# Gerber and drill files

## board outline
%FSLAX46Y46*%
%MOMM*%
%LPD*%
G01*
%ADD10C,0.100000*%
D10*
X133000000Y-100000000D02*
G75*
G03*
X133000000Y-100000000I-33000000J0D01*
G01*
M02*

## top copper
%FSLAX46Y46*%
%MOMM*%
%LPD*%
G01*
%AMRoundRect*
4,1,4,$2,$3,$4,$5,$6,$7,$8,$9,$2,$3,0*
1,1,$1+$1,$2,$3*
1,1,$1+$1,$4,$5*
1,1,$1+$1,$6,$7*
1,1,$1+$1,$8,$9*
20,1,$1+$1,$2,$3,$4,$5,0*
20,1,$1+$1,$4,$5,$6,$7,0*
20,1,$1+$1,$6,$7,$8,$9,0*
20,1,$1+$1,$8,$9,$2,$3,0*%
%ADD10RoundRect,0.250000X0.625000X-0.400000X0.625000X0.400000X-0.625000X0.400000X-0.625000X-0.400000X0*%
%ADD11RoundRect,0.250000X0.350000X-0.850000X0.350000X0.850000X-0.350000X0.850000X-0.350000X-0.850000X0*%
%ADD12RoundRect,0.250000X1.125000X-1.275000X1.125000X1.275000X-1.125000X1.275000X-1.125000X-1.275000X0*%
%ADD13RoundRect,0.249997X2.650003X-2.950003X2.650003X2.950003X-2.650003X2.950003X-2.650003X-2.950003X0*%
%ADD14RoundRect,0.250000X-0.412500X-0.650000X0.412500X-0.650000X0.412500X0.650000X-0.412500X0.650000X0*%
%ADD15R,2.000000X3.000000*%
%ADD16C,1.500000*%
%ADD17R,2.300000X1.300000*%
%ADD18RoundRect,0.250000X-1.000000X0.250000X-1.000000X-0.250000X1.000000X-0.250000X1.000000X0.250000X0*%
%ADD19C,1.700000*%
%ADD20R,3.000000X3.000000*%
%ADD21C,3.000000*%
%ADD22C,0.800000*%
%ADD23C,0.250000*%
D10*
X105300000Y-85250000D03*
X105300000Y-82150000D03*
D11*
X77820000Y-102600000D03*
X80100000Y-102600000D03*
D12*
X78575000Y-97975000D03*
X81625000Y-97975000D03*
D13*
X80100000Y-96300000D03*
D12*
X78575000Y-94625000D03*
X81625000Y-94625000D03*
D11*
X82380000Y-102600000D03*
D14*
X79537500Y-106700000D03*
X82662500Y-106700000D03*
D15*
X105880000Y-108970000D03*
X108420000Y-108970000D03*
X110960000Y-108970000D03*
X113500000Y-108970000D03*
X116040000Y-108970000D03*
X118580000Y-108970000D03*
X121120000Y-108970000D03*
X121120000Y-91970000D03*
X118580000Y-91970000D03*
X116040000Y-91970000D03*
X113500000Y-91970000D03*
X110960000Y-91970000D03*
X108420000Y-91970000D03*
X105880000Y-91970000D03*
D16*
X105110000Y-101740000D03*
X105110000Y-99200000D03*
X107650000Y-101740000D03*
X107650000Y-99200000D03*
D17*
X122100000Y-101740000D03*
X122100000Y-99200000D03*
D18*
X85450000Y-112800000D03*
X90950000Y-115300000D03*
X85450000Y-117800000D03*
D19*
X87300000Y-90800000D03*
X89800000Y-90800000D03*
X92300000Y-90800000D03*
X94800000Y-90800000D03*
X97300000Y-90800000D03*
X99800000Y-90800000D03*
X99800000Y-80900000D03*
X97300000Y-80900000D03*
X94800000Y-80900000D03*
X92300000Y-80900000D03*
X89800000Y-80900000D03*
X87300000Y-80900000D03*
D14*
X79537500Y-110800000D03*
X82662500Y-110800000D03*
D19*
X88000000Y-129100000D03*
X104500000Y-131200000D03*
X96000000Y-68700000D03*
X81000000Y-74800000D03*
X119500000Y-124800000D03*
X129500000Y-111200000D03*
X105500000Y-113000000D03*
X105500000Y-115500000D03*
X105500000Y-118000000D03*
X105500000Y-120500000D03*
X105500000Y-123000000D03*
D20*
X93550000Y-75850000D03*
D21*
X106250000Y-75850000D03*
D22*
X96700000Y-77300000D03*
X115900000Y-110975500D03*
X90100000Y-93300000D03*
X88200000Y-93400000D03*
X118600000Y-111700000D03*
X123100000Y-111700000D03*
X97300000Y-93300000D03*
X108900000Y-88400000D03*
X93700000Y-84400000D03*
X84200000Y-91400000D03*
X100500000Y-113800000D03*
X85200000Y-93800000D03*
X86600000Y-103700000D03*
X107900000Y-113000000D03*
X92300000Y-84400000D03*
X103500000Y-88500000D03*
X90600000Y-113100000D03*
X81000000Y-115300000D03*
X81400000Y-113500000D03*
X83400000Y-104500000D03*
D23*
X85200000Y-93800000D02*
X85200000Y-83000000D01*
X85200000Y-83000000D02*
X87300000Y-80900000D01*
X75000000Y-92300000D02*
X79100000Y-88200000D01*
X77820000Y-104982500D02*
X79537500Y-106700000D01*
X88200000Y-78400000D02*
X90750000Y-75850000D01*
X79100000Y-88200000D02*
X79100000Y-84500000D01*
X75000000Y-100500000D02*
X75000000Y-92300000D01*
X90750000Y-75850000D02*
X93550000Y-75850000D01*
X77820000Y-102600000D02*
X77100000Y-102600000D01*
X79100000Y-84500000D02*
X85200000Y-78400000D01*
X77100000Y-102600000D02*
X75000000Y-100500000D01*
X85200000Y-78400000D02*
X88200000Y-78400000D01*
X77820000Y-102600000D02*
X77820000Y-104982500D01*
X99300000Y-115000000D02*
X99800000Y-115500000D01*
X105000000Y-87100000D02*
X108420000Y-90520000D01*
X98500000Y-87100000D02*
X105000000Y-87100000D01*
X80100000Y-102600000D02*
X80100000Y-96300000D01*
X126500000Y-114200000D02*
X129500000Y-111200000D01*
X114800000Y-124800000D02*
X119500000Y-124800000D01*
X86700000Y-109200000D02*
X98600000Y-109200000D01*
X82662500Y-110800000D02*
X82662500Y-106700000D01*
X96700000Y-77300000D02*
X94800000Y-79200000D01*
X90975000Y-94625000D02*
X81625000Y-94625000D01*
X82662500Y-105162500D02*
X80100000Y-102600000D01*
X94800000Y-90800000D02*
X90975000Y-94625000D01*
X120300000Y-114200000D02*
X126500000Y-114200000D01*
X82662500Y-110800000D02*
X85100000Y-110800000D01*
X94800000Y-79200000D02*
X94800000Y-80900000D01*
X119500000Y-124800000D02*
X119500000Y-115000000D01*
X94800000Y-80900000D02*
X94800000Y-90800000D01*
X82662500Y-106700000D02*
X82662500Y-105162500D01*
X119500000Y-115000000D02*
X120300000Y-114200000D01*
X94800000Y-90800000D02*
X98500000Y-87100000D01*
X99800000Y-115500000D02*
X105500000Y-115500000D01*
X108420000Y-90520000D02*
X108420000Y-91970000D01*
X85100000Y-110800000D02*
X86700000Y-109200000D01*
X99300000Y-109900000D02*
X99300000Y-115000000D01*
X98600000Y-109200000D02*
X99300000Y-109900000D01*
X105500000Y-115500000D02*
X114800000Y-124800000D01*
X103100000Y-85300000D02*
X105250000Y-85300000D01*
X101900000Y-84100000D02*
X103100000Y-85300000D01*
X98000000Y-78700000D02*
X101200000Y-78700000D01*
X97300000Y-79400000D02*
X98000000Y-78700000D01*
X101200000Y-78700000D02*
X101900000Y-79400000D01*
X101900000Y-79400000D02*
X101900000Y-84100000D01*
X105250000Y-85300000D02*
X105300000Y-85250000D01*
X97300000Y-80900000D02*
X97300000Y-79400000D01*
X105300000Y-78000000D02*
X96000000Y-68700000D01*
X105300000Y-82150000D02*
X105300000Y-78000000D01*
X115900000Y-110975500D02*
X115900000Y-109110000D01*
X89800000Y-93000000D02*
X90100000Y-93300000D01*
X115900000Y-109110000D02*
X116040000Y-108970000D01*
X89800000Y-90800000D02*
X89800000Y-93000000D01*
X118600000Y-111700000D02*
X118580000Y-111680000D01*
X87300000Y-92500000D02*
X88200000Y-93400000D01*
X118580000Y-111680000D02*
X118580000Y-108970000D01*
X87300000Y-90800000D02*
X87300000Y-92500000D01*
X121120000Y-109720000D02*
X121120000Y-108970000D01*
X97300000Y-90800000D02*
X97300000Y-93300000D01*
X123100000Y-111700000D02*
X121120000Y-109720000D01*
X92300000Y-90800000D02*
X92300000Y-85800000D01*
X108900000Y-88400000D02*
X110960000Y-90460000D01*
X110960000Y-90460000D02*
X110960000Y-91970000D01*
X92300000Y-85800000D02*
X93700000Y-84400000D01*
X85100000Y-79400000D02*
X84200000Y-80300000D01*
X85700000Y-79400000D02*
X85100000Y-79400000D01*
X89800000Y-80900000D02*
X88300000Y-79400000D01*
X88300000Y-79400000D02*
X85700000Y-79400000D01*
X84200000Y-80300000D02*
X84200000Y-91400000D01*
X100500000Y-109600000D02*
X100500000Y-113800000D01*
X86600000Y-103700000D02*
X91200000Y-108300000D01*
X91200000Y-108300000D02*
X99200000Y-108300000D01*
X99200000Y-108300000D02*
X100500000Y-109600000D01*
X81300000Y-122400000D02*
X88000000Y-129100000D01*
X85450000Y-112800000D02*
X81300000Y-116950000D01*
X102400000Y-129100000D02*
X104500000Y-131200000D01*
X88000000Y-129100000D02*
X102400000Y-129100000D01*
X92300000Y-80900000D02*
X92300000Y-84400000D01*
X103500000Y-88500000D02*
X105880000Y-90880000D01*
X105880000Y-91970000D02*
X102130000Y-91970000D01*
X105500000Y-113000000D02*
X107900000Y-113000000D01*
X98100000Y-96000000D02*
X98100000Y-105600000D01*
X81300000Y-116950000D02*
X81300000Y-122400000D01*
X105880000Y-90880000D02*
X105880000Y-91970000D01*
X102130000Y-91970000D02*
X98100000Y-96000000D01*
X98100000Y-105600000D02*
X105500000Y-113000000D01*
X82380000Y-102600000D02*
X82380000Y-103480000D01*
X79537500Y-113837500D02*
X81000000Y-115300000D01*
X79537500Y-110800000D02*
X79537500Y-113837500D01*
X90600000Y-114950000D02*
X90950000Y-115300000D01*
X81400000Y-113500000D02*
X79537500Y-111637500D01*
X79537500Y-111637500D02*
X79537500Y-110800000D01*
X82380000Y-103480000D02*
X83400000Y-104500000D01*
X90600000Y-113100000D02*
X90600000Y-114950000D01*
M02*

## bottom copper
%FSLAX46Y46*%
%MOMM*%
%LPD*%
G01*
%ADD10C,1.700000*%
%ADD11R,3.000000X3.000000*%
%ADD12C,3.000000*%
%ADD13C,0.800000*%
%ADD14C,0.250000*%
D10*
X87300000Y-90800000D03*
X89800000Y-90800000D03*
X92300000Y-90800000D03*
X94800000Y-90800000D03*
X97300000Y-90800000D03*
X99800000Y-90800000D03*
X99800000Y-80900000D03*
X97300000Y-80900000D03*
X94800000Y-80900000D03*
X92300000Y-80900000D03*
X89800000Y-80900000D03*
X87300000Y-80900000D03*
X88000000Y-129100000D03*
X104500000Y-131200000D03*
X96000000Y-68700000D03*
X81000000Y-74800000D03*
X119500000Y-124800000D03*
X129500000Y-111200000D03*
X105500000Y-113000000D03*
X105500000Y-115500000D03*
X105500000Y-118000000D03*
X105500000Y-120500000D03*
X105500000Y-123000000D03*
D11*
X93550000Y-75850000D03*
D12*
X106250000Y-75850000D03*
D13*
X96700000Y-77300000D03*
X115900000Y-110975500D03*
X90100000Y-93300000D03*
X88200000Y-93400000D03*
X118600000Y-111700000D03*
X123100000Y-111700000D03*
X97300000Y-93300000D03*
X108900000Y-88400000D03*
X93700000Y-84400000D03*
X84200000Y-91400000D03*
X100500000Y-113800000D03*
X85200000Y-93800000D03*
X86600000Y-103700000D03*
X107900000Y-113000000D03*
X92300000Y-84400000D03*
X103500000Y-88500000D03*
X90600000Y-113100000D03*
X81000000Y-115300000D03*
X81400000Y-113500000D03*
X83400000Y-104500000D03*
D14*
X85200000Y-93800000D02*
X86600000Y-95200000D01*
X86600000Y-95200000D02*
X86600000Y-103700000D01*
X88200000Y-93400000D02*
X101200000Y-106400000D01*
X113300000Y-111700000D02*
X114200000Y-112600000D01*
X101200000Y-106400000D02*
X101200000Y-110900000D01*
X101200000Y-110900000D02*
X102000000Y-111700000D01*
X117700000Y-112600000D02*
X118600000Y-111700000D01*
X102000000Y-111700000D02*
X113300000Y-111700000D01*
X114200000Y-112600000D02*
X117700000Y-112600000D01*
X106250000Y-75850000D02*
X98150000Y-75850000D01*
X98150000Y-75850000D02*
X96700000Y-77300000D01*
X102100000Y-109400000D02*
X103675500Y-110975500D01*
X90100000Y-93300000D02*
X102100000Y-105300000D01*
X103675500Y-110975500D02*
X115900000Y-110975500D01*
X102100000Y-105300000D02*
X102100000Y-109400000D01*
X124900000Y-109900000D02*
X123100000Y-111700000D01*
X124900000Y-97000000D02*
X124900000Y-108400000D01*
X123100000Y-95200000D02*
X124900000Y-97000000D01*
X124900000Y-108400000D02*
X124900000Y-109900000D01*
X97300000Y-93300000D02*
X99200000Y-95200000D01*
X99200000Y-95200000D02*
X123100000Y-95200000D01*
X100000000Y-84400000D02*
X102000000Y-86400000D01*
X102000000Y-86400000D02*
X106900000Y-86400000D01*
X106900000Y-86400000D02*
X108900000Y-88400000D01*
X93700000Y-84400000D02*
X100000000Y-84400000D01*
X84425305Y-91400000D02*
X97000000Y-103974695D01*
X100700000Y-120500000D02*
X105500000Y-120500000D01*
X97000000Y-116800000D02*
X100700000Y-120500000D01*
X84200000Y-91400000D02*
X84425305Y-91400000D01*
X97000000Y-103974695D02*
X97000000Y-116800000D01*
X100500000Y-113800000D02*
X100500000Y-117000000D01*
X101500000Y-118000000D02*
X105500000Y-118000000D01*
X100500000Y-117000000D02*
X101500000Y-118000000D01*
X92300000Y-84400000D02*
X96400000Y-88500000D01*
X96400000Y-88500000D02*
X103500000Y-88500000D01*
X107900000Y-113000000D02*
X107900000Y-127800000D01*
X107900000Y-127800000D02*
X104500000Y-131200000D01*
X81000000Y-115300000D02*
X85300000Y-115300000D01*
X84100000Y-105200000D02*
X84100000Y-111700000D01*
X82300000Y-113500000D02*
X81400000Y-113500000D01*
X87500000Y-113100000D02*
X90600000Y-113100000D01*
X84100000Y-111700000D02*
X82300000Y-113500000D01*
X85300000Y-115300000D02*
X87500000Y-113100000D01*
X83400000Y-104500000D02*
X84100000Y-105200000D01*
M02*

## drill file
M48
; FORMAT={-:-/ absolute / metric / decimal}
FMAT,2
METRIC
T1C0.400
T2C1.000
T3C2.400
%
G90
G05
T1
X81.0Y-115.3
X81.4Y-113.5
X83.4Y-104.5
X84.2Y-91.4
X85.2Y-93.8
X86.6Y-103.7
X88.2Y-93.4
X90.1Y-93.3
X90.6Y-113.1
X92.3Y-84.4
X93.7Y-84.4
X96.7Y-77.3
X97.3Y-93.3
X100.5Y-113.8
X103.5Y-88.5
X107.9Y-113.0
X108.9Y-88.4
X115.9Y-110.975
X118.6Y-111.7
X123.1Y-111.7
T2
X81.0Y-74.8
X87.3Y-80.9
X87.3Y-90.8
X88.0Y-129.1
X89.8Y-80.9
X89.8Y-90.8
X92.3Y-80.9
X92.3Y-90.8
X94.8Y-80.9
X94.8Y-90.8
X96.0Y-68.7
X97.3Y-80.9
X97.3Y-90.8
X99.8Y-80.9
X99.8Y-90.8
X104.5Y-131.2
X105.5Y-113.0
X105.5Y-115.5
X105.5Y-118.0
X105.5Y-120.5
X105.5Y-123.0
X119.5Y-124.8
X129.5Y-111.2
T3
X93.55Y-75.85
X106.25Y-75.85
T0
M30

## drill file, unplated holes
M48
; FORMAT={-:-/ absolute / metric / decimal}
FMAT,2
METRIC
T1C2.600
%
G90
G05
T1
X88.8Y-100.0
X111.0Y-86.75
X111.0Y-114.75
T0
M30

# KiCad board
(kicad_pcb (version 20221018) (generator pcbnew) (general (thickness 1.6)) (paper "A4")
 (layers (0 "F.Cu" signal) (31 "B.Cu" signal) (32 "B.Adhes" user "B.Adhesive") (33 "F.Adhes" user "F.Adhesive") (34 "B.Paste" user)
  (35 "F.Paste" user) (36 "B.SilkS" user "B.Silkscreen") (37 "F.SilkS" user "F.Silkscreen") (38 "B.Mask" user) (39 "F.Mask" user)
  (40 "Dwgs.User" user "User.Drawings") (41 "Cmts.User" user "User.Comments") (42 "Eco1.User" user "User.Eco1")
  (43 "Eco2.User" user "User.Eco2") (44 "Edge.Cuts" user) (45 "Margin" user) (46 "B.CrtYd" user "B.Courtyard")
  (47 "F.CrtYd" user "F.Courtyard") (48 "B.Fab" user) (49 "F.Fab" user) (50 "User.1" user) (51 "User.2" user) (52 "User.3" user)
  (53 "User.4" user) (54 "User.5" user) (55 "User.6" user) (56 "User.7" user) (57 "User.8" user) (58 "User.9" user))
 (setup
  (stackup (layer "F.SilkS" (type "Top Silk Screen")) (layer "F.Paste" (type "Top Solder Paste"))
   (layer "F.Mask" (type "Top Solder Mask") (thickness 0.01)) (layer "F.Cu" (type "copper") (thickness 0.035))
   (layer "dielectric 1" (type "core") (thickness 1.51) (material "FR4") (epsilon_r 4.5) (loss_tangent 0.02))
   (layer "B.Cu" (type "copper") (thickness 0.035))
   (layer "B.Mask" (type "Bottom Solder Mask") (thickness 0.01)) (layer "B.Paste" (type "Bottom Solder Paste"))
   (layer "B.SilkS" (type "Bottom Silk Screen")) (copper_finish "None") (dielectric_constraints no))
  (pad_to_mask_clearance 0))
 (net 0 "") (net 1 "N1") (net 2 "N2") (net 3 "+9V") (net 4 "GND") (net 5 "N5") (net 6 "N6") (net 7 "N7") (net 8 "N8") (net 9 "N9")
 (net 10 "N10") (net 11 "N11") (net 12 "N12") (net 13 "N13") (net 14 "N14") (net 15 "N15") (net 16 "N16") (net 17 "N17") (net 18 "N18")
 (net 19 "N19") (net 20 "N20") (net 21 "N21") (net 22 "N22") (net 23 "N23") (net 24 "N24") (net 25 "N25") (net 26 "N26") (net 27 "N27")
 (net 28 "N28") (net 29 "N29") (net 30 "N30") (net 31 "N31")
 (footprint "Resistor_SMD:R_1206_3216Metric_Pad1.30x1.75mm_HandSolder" (layer "F.Cu") (at 105.3 83.7 90)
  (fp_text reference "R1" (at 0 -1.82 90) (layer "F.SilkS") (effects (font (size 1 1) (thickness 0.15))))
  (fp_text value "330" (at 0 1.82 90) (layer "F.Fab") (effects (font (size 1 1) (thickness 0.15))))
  (pad "1" smd roundrect (at -1.55 0 90) (size 1.3 1.75) (layers "F.Cu" "F.Paste" "F.Mask") (roundrect_rratio 0.1923076923) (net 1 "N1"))
  (pad "2" smd roundrect (at 1.55 0 90) (size 1.3 1.75) (layers "F.Cu" "F.Paste" "F.Mask") (roundrect_rratio 0.1923076923) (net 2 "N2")))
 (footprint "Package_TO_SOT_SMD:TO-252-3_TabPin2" (layer "F.Cu") (at 80.1 97.56 90)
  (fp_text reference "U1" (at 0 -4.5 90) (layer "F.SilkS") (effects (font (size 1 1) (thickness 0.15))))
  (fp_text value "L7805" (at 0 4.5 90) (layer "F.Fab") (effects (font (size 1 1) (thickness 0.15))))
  (pad "1" smd roundrect (at -5.04 -2.28 90) (size 2.2 1.2) (layers "F.Cu" "F.Paste" "F.Mask") (roundrect_rratio 0.2083333333) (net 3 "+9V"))
  (pad "2" smd roundrect (at -5.04 0 90) (size 2.2 1.2) (layers "F.Cu" "F.Paste" "F.Mask") (roundrect_rratio 0.2083333333) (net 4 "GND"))
  (pad "2" smd roundrect (at -0.415 -1.525 90) (size 3.05 2.75) (layers "F.Cu" "F.Paste") (roundrect_rratio 0.09090909091) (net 4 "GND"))
  (pad "2" smd roundrect (at -0.415 1.525 90) (size 3.05 2.75) (layers "F.Cu" "F.Paste") (roundrect_rratio 0.09090909091) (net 4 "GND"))
  (pad "2" smd roundrect (at 1.26 0 90) (size 6.4 5.8) (layers "F.Cu" "F.Mask") (roundrect_rratio 0.04310293103) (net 4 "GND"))
  (pad "2" smd roundrect (at 2.935 -1.525 90) (size 3.05 2.75) (layers "F.Cu" "F.Paste") (roundrect_rratio 0.09090909091) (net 4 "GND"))
  (pad "2" smd roundrect (at 2.935 1.525 90) (size 3.05 2.75) (layers "F.Cu" "F.Paste") (roundrect_rratio 0.09090909091) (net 4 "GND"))
  (pad "3" smd roundrect (at -5.04 2.28 90) (size 2.2 1.2) (layers "F.Cu" "F.Paste" "F.Mask") (roundrect_rratio 0.2083333333) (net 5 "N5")))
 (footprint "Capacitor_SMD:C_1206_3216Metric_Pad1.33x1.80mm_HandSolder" (layer "F.Cu") (at 81.1 106.7)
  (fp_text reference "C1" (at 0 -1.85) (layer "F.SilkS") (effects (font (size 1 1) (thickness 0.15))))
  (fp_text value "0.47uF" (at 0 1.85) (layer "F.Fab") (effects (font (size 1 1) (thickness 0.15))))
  (pad "1" smd roundrect (at -1.5625 0) (size 1.325 1.8) (layers "F.Cu" "F.Paste" "F.Mask") (roundrect_rratio 0.1886792453) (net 3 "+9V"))
  (pad "2" smd roundrect (at 1.5625 0) (size 1.325 1.8) (layers "F.Cu" "F.Paste" "F.Mask") (roundrect_rratio 0.1886792453) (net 4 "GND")))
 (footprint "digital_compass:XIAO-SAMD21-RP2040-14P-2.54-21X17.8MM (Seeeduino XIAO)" (layer "F.Cu") (at 113.5 100.47 90)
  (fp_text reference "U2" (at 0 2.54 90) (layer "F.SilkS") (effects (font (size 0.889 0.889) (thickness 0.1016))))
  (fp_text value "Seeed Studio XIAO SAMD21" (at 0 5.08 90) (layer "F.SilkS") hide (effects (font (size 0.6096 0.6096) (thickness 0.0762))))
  (pad "1" smd rect (at -8.5 -7.62 90) (size 3 2) (layers "F.Cu" "F.Paste" "F.Mask") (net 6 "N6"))
  (pad "2" smd rect (at -8.5 -5.08 90) (size 3 2) (layers "F.Cu" "F.Paste" "F.Mask") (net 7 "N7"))
  (pad "3" smd rect (at -8.5 -2.54 90) (size 3 2) (layers "F.Cu" "F.Paste" "F.Mask") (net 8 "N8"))
  (pad "4" smd rect (at -8.5 0 90) (size 3 2) (layers "F.Cu" "F.Paste" "F.Mask") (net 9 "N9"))
  (pad "5" smd rect (at -8.5 2.54 90) (size 3 2) (layers "F.Cu" "F.Paste" "F.Mask") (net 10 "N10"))
  (pad "6" smd rect (at -8.5 5.08 270) (size 3 2) (layers "F.Cu" "F.Paste" "F.Mask") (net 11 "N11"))
  (pad "7" smd rect (at -8.5 7.62 90) (size 3 2) (layers "F.Cu" "F.Paste" "F.Mask") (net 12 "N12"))
  (pad "8" smd rect (at 8.5 7.62 90) (size 3 2) (layers "F.Cu" "F.Paste" "F.Mask") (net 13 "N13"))
  (pad "9" smd rect (at 8.5 5.08 90) (size 3 2) (layers "F.Cu" "F.Paste" "F.Mask") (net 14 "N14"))
  (pad "10" smd rect (at 8.5 2.54 90) (size 3 2) (layers "F.Cu" "F.Paste" "F.Mask") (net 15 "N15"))
  (pad "11" smd rect (at 8.5 0 90) (size 3 2) (layers "F.Cu" "F.Paste" "F.Mask") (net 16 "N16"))
  (pad "12" smd rect (at 8.5 -2.54 90) (size 3 2) (layers "F.Cu" "F.Paste" "F.Mask") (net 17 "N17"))
  (pad "13" smd rect (at 8.5 -5.08 90) (size 3 2) (layers "F.Cu" "F.Paste" "F.Mask") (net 4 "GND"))
  (pad "14" smd rect (at 8.5 -7.62 90) (size 3 2) (layers "F.Cu" "F.Paste" "F.Mask") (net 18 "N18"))
  (pad "15" smd circle (at -1.27 -8.39 180) (size 1.5 1.5) (layers "F.Cu" "F.Paste" "F.Mask") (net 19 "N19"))
  (pad "16" smd circle (at 1.27 -8.39 180) (size 1.5 1.5) (layers "F.Cu" "F.Paste" "F.Mask") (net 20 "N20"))
  (pad "17" smd circle (at -1.27 -5.85 180) (size 1.5 1.5) (layers "F.Cu" "F.Paste" "F.Mask") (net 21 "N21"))
  (pad "18" smd circle (at 1.27 -5.85 180) (size 1.5 1.5) (layers "F.Cu" "F.Paste" "F.Mask") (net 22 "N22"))
  (pad "19" smd rect (at -1.27 8.6 180) (size 2.3 1.3) (layers "F.Cu" "F.Paste" "F.Mask") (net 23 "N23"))
  (pad "20" smd rect (at 1.27 8.6 180) (size 2.3 1.3) (layers "F.Cu" "F.Paste" "F.Mask") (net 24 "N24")))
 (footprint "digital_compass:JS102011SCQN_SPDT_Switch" (layer "F.Cu") (at 88.2 115.3 -90)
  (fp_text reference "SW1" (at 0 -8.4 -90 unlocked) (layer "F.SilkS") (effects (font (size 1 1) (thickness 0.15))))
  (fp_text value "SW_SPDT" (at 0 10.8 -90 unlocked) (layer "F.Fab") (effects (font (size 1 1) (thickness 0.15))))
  (pad "1" smd roundrect (at -2.5 2.75 270) (size 1 2.5) (layers "F.Cu" "F.Paste" "F.Mask") (roundrect_rratio 0.25) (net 18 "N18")
   (thermal_bridge_angle 45))
  (pad "2" smd roundrect (at 0 -2.75 270) (size 1 2.5) (layers "F.Cu" "F.Paste" "F.Mask") (roundrect_rratio 0.25) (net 5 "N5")
   (thermal_bridge_angle 45))
  (pad "3" smd roundrect (at 2.5 2.75 270) (size 1 2.5) (layers "F.Cu" "F.Paste" "F.Mask") (roundrect_rratio 0.25) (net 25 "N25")
   (thermal_bridge_angle 45)))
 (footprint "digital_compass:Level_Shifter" (layer "F.Cu") (at 93.55 85.85)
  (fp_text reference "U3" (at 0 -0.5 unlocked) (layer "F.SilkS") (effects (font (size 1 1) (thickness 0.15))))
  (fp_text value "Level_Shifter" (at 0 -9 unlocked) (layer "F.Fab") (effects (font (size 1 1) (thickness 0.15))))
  (pad "1" thru_hole circle (at -6.25 4.95) (size 1.7 1.7) (drill 1) (layers "*.Cu" "*.Mask") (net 11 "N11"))
  (pad "2" thru_hole circle (at -3.75 4.95) (size 1.7 1.7) (drill 1) (layers "*.Cu" "*.Mask") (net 10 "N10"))
  (pad "3" thru_hole circle (at -1.25 4.95) (size 1.7 1.7) (drill 1) (layers "*.Cu" "*.Mask") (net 17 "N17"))
  (pad "4" thru_hole circle (at 1.25 4.95) (size 1.7 1.7) (drill 1) (layers "*.Cu" "*.Mask") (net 4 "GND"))
  (pad "5" thru_hole circle (at 3.75 4.95) (size 1.7 1.7) (drill 1) (layers "*.Cu" "*.Mask") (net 12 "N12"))
  (pad "6" thru_hole circle (at 6.25 4.95) (size 1.7 1.7) (drill 1) (layers "*.Cu" "*.Mask") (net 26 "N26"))
  (pad "7" thru_hole circle (at 6.25 -4.95) (size 1.7 1.7) (drill 1) (layers "*.Cu" "*.Mask") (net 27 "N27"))
  (pad "8" thru_hole circle (at 3.75 -4.95) (size 1.7 1.7) (drill 1) (layers "*.Cu" "*.Mask") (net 1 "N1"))
  (pad "9" thru_hole circle (at 1.25 -4.95) (size 1.7 1.7) (drill 1) (layers "*.Cu" "*.Mask") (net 4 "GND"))
  (pad "10" thru_hole circle (at -1.25 -4.95) (size 1.7 1.7) (drill 1) (layers "*.Cu" "*.Mask") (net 18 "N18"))
  (pad "11" thru_hole circle (at -3.75 -4.95) (size 1.7 1.7) (drill 1) (layers "*.Cu" "*.Mask") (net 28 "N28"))
  (pad "12" thru_hole circle (at -6.25 -4.95) (size 1.7 1.7) (drill 1) (layers "*.Cu" "*.Mask") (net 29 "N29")))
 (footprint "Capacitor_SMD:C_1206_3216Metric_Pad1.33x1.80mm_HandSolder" (layer "F.Cu") (at 81.1 110.8)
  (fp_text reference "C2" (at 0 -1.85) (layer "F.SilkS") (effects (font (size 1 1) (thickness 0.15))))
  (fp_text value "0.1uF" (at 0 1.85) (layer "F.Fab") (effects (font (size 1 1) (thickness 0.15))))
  (pad "1" smd roundrect (at -1.5625 0) (size 1.325 1.8) (layers "F.Cu" "F.Paste" "F.Mask") (roundrect_rratio 0.1886792453) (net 5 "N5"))
  (pad "2" smd roundrect (at 1.5625 0) (size 1.325 1.8) (layers "F.Cu" "F.Paste" "F.Mask") (roundrect_rratio 0.1886792453) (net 4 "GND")))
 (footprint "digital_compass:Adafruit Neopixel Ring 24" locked (layer "F.Cu") (at 100 100)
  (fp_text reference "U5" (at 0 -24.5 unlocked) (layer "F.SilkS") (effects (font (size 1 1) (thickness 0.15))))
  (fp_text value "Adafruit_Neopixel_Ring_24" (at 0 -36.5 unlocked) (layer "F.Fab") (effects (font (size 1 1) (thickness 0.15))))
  (pad "1" thru_hole circle locked (at -12 29.1) (size 1.7 1.7) (drill 1) (layers "*.Cu" "*.Mask") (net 18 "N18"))
  (pad "2" thru_hole circle locked (at 4.5 31.2) (size 1.7 1.7) (drill 1) (layers "*.Cu" "*.Mask") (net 18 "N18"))
  (pad "3" thru_hole circle locked (at -4 -31.3) (size 1.7 1.7) (drill 1) (layers "*.Cu" "*.Mask") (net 2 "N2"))
  (pad "4" thru_hole circle locked (at -19 -25.2) (size 1.7 1.7) (drill 1) (layers "*.Cu" "*.Mask") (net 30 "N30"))
  (pad "5" thru_hole circle locked (at 19.5 24.8) (size 1.7 1.7) (drill 1) (layers "*.Cu" "*.Mask") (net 4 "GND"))
  (pad "6" thru_hole circle locked (at 29.5 11.2) (size 1.7 1.7) (drill 1) (layers "*.Cu" "*.Mask") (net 4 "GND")))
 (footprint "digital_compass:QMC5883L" (layer "F.Cu") (at 100 118)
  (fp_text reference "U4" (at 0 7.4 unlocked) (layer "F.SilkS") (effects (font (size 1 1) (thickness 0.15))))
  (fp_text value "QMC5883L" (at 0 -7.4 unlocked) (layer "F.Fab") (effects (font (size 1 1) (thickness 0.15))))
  (pad "1" thru_hole circle (at 5.5 -5) (size 1.7 1.7) (drill 1) (layers "*.Cu" "*.Mask") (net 18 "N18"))
  (pad "2" thru_hole circle (at 5.5 -2.5) (size 1.7 1.7) (drill 1) (layers "*.Cu" "*.Mask") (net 4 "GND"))
  (pad "3" thru_hole circle (at 5.5 0) (size 1.7 1.7) (drill 1) (layers "*.Cu" "*.Mask") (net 29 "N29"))
  (pad "4" thru_hole circle (at 5.5 2.5) (size 1.7 1.7) (drill 1) (layers "*.Cu" "*.Mask") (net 28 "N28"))
  (pad "5" thru_hole circle (at 5.5 5) (size 1.7 1.7) (drill 1) (layers "*.Cu" "*.Mask") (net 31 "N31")))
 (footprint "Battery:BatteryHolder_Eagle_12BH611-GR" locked (layer "B.Cu") (at 93.55 75.85 90)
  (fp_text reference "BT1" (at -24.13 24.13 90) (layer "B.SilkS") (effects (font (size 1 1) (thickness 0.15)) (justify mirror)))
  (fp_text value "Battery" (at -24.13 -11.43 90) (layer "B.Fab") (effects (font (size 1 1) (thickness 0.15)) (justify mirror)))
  (pad "" np_thru_hole circle locked (at -38.9 17.45 90) (size 2.6 2.6) (drill 2.6) (layers "*.Cu" "*.Mask"))
  (pad "" np_thru_hole circle locked (at -24.15 -4.75 90) (size 2.6 2.6) (drill 2.6) (layers "*.Cu" "*.Mask"))
  (pad "" np_thru_hole circle locked (at -10.9 17.45 90) (size 2.6 2.6) (drill 2.6) (layers "*.Cu" "*.Mask"))
  (pad "1" thru_hole rect locked (at 0 0 90) (size 3 3) (drill 2.4) (layers "*.Cu" "*.Mask") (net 3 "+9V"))
  (pad "2" thru_hole circle locked (at 0 12.7 90) (size 3 3) (drill 2.4) (layers "*.Cu" "*.Mask") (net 4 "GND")))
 (gr_circle (center 100 100) (end 133 100) (stroke (width 0.1) (type default)) (fill none) (layer "Edge.Cuts"))
 (segment (start 75 92.3) (end 79.1 88.2) (width 0.25) (layer "F.Cu") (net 3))
 (segment (start 77.82 104.9825) (end 79.5375 106.7) (width 0.25) (layer "F.Cu") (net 3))
 (segment (start 88.2 78.4) (end 90.75 75.85) (width 0.25) (layer "F.Cu") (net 3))
 (segment (start 79.1 88.2) (end 79.1 84.5) (width 0.25) (layer "F.Cu") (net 3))
 (segment (start 75 100.5) (end 75 92.3) (width 0.25) (layer "F.Cu") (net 3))
 (segment (start 90.75 75.85) (end 93.55 75.85) (width 0.25) (layer "F.Cu") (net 3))
 (segment (start 77.82 102.6) (end 77.1 102.6) (width 0.25) (layer "F.Cu") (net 3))
 (segment (start 79.1 84.5) (end 85.2 78.4) (width 0.25) (layer "F.Cu") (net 3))
 (segment (start 77.1 102.6) (end 75 100.5) (width 0.25) (layer "F.Cu") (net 3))
 (segment (start 85.2 78.4) (end 88.2 78.4) (width 0.25) (layer "F.Cu") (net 3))
 (segment (start 77.82 102.6) (end 77.82 104.9825) (width 0.25) (layer "F.Cu") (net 3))
 (segment (start 99.3 115) (end 99.8 115.5) (width 0.25) (layer "F.Cu") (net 4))
 (segment (start 105 87.1) (end 108.42 90.52) (width 0.25) (layer "F.Cu") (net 4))
 (segment (start 98.5 87.1) (end 105 87.1) (width 0.25) (layer "F.Cu") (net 4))
 (segment (start 80.1 102.6) (end 80.1 96.3) (width 0.25) (layer "F.Cu") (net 4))
 (segment (start 126.5 114.2) (end 129.5 111.2) (width 0.25) (layer "F.Cu") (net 4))
 (segment (start 114.8 124.8) (end 119.5 124.8) (width 0.25) (layer "F.Cu") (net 4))
 (segment (start 86.7 109.2) (end 98.6 109.2) (width 0.25) (layer "F.Cu") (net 4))
 (segment (start 82.6625 110.8) (end 82.6625 106.7) (width 0.25) (layer "F.Cu") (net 4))
 (segment (start 96.7 77.3) (end 94.8 79.2) (width 0.25) (layer "F.Cu") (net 4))
 (segment (start 90.975 94.625) (end 81.625 94.625) (width 0.25) (layer "F.Cu") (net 4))
 (segment (start 82.6625 105.1625) (end 80.1 102.6) (width 0.25) (layer "F.Cu") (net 4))
 (segment (start 94.8 90.8) (end 90.975 94.625) (width 0.25) (layer "F.Cu") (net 4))
 (segment (start 120.3 114.2) (end 126.5 114.2) (width 0.25) (layer "F.Cu") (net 4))
 (segment (start 82.6625 110.8) (end 85.1 110.8) (width 0.25) (layer "F.Cu") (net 4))
 (segment (start 94.8 79.2) (end 94.8 80.9) (width 0.25) (layer "F.Cu") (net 4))
 (segment (start 119.5 124.8) (end 119.5 115) (width 0.25) (layer "F.Cu") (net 4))
 (segment (start 94.8 80.9) (end 94.8 90.8) (width 0.25) (layer "F.Cu") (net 4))
 (segment (start 82.6625 106.7) (end 82.6625 105.1625) (width 0.25) (layer "F.Cu") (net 4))
 (segment (start 119.5 115) (end 120.3 114.2) (width 0.25) (layer "F.Cu") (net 4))
 (segment (start 94.8 90.8) (end 98.5 87.1) (width 0.25) (layer "F.Cu") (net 4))
 (segment (start 99.8 115.5) (end 105.5 115.5) (width 0.25) (layer "F.Cu") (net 4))
 (segment (start 108.42 90.52) (end 108.42 91.97) (width 0.25) (layer "F.Cu") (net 4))
 (segment (start 85.1 110.8) (end 86.7 109.2) (width 0.25) (layer "F.Cu") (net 4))
 (segment (start 99.3 109.9) (end 99.3 115) (width 0.25) (layer "F.Cu") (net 4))
 (segment (start 98.6 109.2) (end 99.3 109.9) (width 0.25) (layer "F.Cu") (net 4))
 (segment (start 105.5 115.5) (end 114.8 124.8) (width 0.25) (layer "F.Cu") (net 4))
 (via (at 96.7 77.3) (size 0.8) (drill 0.4) (layers "F.Cu" "B.Cu") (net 4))
 (segment (start 106.25 75.85) (end 98.15 75.85) (width 0.25) (layer "B.Cu") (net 4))
 (segment (start 98.15 75.85) (end 96.7 77.3) (width 0.25) (layer "B.Cu") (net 4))
 (segment (start 103.1 85.3) (end 105.25 85.3) (width 0.25) (layer "F.Cu") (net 1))
 (segment (start 101.9 84.1) (end 103.1 85.3) (width 0.25) (layer "F.Cu") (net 1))
 (segment (start 98 78.7) (end 101.2 78.7) (width 0.25) (layer "F.Cu") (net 1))
 (segment (start 97.3 79.4) (end 98 78.7) (width 0.25) (layer "F.Cu") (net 1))
 (segment (start 101.2 78.7) (end 101.9 79.4) (width 0.25) (layer "F.Cu") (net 1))
 (segment (start 101.9 79.4) (end 101.9 84.1) (width 0.25) (layer "F.Cu") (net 1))
 (segment (start 105.25 85.3) (end 105.3 85.25) (width 0.25) (layer "F.Cu") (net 1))
 (segment (start 97.3 80.9) (end 97.3 79.4) (width 0.25) (layer "F.Cu") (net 1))
 (segment (start 105.3 78) (end 96 68.7) (width 0.25) (layer "F.Cu") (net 2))
 (segment (start 105.3 82.15) (end 105.3 78) (width 0.25) (layer "F.Cu") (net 2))
 (segment (start 115.9 110.9755) (end 115.9 109.11) (width 0.25) (layer "F.Cu") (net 10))
 (segment (start 89.8 93) (end 90.1 93.3) (width 0.25) (layer "F.Cu") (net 10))
 (segment (start 115.9 109.11) (end 116.04 108.97) (width 0.25) (layer "F.Cu") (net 10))
 (segment (start 89.8 90.8) (end 89.8 93) (width 0.25) (layer "F.Cu") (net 10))
 (via (at 115.9 110.9755) (size 0.8) (drill 0.4) (layers "F.Cu" "B.Cu") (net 10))
 (via (at 90.1 93.3) (size 0.8) (drill 0.4) (layers "F.Cu" "B.Cu") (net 10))
 (segment (start 102.1 109.4) (end 103.6755 110.9755) (width 0.25) (layer "B.Cu") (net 10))
 (segment (start 90.1 93.3) (end 102.1 105.3) (width 0.25) (layer "B.Cu") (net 10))
 (segment (start 103.6755 110.9755) (end 115.9 110.9755) (width 0.25) (layer "B.Cu") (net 10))
 (segment (start 102.1 105.3) (end 102.1 109.4) (width 0.25) (layer "B.Cu") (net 10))
 (segment (start 118.6 111.7) (end 118.58 111.68) (width 0.25) (layer "F.Cu") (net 11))
 (segment (start 87.3 92.5) (end 88.2 93.4) (width 0.25) (layer "F.Cu") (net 11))
 (segment (start 118.58 111.68) (end 118.58 108.97) (width 0.25) (layer "F.Cu") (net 11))
 (segment (start 87.3 90.8) (end 87.3 92.5) (width 0.25) (layer "F.Cu") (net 11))
 (via (at 88.2 93.4) (size 0.8) (drill 0.4) (layers "F.Cu" "B.Cu") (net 11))
 (via (at 118.6 111.7) (size 0.8) (drill 0.4) (layers "F.Cu" "B.Cu") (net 11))
 (segment (start 117.7 112.6) (end 118.6 111.7) (width 0.25) (layer "B.Cu") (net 11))
 (segment (start 101.2 106.4) (end 101.2 110.9) (width 0.25) (layer "B.Cu") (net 11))
 (segment (start 114.2 112.6) (end 117.7 112.6) (width 0.25) (layer "B.Cu") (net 11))
 (segment (start 101.2 110.9) (end 102 111.7) (width 0.25) (layer "B.Cu") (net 11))
 (segment (start 113.3 111.7) (end 114.2 112.6) (width 0.25) (layer "B.Cu") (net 11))
 (segment (start 88.2 93.4) (end 101.2 106.4) (width 0.25) (layer "B.Cu") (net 11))
 (segment (start 102 111.7) (end 113.3 111.7) (width 0.25) (layer "B.Cu") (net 11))
 (segment (start 121.12 109.72) (end 121.12 108.97) (width 0.25) (layer "F.Cu") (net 12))
 (segment (start 97.3 90.8) (end 97.3 93.3) (width 0.25) (layer "F.Cu") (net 12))
 (segment (start 123.1 111.7) (end 121.12 109.72) (width 0.25) (layer "F.Cu") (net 12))
 (via (at 123.1 111.7) (size 0.8) (drill 0.4) (layers "F.Cu" "B.Cu") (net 12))
 (via (at 97.3 93.3) (size 0.8) (drill 0.4) (layers "F.Cu" "B.Cu") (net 12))
 (segment (start 124.9 109.9) (end 123.1 111.7) (width 0.25) (layer "B.Cu") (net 12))
 (segment (start 124.9 97) (end 124.9 108.4) (width 0.25) (layer "B.Cu") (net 12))
 (segment (start 123.1 95.2) (end 124.9 97) (width 0.25) (layer "B.Cu") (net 12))
 (segment (start 124.9 108.4) (end 124.9 109.9) (width 0.25) (layer "B.Cu") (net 12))
 (segment (start 97.3 93.3) (end 99.2 95.2) (width 0.25) (layer "B.Cu") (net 12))
 (segment (start 99.2 95.2) (end 123.1 95.2) (width 0.25) (layer "B.Cu") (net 12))
 (segment (start 92.3 90.8) (end 92.3 85.8) (width 0.25) (layer "F.Cu") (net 17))
 (segment (start 108.9 88.4) (end 110.96 90.46) (width 0.25) (layer "F.Cu") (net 17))
 (segment (start 110.96 90.46) (end 110.96 91.97) (width 0.25) (layer "F.Cu") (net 17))
 (segment (start 92.3 85.8) (end 93.7 84.4) (width 0.25) (layer "F.Cu") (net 17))
 (via (at 108.9 88.4) (size 0.8) (drill 0.4) (layers "F.Cu" "B.Cu") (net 17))
 (via (at 93.7 84.4) (size 0.8) (drill 0.4) (layers "F.Cu" "B.Cu") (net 17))
 (segment (start 100 84.4) (end 102 86.4) (width 0.25) (layer "B.Cu") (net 17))
 (segment (start 102 86.4) (end 106.9 86.4) (width 0.25) (layer "B.Cu") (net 17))
 (segment (start 106.9 86.4) (end 108.9 88.4) (width 0.25) (layer "B.Cu") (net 17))
 (segment (start 93.7 84.4) (end 100 84.4) (width 0.25) (layer "B.Cu") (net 17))
 (segment (start 85.1 79.4) (end 84.2 80.3) (width 0.25) (layer "F.Cu") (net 28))
 (segment (start 85.7 79.4) (end 85.1 79.4) (width 0.25) (layer "F.Cu") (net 28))
 (segment (start 89.8 80.9) (end 88.3 79.4) (width 0.25) (layer "F.Cu") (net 28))
 (segment (start 88.3 79.4) (end 85.7 79.4) (width 0.25) (layer "F.Cu") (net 28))
 (segment (start 84.2 80.3) (end 84.2 91.4) (width 0.25) (layer "F.Cu") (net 28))
 (via (at 84.2 91.4) (size 0.8) (drill 0.4) (layers "F.Cu" "B.Cu") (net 28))
 (segment (start 84.425305 91.4) (end 97 103.974695) (width 0.25) (layer "B.Cu") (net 28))
 (segment (start 100.7 120.5) (end 105.5 120.5) (width 0.25) (layer "B.Cu") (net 28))
 (segment (start 97 116.8) (end 100.7 120.5) (width 0.25) (layer "B.Cu") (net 28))
 (segment (start 84.2 91.4) (end 84.425305 91.4) (width 0.25) (layer "B.Cu") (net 28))
 (segment (start 97 103.974695) (end 97 116.8) (width 0.25) (layer "B.Cu") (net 28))
 (segment (start 100.5 109.6) (end 100.5 113.8) (width 0.25) (layer "F.Cu") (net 29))
 (segment (start 86.6 103.7) (end 91.2 108.3) (width 0.25) (layer "F.Cu") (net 29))
 (segment (start 91.2 108.3) (end 99.2 108.3) (width 0.25) (layer "F.Cu") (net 29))
 (segment (start 99.2 108.3) (end 100.5 109.6) (width 0.25) (layer "F.Cu") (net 29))
 (segment (start 85.2 93.8) (end 85.2 83) (width 0.25) (layer "F.Cu") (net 29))
 (segment (start 85.2 83) (end 87.3 80.9) (width 0.25) (layer "F.Cu") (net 29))
 (via (at 100.5 113.8) (size 0.8) (drill 0.4) (layers "F.Cu" "B.Cu") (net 29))
 (via (at 85.2 93.8) (size 0.8) (drill 0.4) (layers "F.Cu" "B.Cu") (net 29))
 (via (at 86.6 103.7) (size 0.8) (drill 0.4) (layers "F.Cu" "B.Cu") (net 29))
 (segment (start 85.2 93.8) (end 86.6 95.2) (width 0.25) (layer "B.Cu") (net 29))
 (segment (start 100.5 113.8) (end 100.5 117) (width 0.25) (layer "B.Cu") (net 29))
 (segment (start 101.5 118) (end 105.5 118) (width 0.25) (layer "B.Cu") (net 29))
 (segment (start 100.5 117) (end 101.5 118) (width 0.25) (layer "B.Cu") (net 29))
 (segment (start 86.6 95.2) (end 86.6 103.7) (width 0.25) (layer "B.Cu") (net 29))
 (segment (start 81.3 122.4) (end 88 129.1) (width 0.25) (layer "F.Cu") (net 18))
 (segment (start 85.45 112.8) (end 81.3 116.95) (width 0.25) (layer "F.Cu") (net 18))
 (segment (start 102.4 129.1) (end 104.5 131.2) (width 0.25) (layer "F.Cu") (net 18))
 (segment (start 88 129.1) (end 102.4 129.1) (width 0.25) (layer "F.Cu") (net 18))
 (segment (start 92.3 80.9) (end 92.3 84.4) (width 0.25) (layer "F.Cu") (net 18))
 (segment (start 103.5 88.5) (end 105.88 90.88) (width 0.25) (layer "F.Cu") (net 18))
 (segment (start 105.88 91.97) (end 102.13 91.97) (width 0.25) (layer "F.Cu") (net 18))
 (segment (start 105.5 113) (end 107.9 113) (width 0.25) (layer "F.Cu") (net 18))
 (segment (start 98.1 96) (end 98.1 105.6) (width 0.25) (layer "F.Cu") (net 18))
 (segment (start 81.3 116.95) (end 81.3 122.4) (width 0.25) (layer "F.Cu") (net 18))
 (segment (start 105.88 90.88) (end 105.88 91.97) (width 0.25) (layer "F.Cu") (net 18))
 (segment (start 102.13 91.97) (end 98.1 96) (width 0.25) (layer "F.Cu") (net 18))
 (segment (start 98.1 105.6) (end 105.5 113) (width 0.25) (layer "F.Cu") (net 18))
 (via (at 107.9 113) (size 0.8) (drill 0.4) (layers "F.Cu" "B.Cu") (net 18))
 (via (at 92.3 84.4) (size 0.8) (drill 0.4) (layers "F.Cu" "B.Cu") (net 18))
 (via (at 103.5 88.5) (size 0.8) (drill 0.4) (layers "F.Cu" "B.Cu") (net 18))
 (segment (start 92.3 84.4) (end 96.4 88.5) (width 0.25) (layer "B.Cu") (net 18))
 (segment (start 96.4 88.5) (end 103.5 88.5) (width 0.25) (layer "B.Cu") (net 18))
 (segment (start 107.9 113) (end 107.9 127.8) (width 0.25) (layer "B.Cu") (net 18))
 (segment (start 107.9 127.8) (end 104.5 131.2) (width 0.25) (layer "B.Cu") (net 18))
 (segment (start 82.38 102.6) (end 82.38 103.48) (width 0.25) (layer "F.Cu") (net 5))
 (segment (start 79.5375 113.8375) (end 81 115.3) (width 0.25) (layer "F.Cu") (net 5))
 (segment (start 79.5375 110.8) (end 79.5375 113.8375) (width 0.25) (layer "F.Cu") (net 5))
 (segment (start 90.6 114.95) (end 90.95 115.3) (width 0.25) (layer "F.Cu") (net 5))
 (segment (start 81.4 113.5) (end 79.5375 111.6375) (width 0.25) (layer "F.Cu") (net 5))
 (segment (start 79.5375 111.6375) (end 79.5375 110.8) (width 0.25) (layer "F.Cu") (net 5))
 (segment (start 82.38 103.48) (end 83.4 104.5) (width 0.25) (layer "F.Cu") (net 5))
 (segment (start 90.6 113.1) (end 90.6 114.95) (width 0.25) (layer "F.Cu") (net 5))
 (via (at 90.6 113.1) (size 0.8) (drill 0.4) (layers "F.Cu" "B.Cu") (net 5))
 (via (at 81 115.3) (size 0.8) (drill 0.4) (layers "F.Cu" "B.Cu") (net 5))
 (via (at 81.4 113.5) (size 0.8) (drill 0.4) (layers "F.Cu" "B.Cu") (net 5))
 (via (at 83.4 104.5) (size 0.8) (drill 0.4) (layers "F.Cu" "B.Cu") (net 5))
 (segment (start 81 115.3) (end 85.3 115.3) (width 0.25) (layer "B.Cu") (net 5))
 (segment (start 84.1 105.2) (end 84.1 111.7) (width 0.25) (layer "B.Cu") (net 5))
 (segment (start 82.3 113.5) (end 81.4 113.5) (width 0.25) (layer "B.Cu") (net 5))
 (segment (start 87.5 113.1) (end 90.6 113.1) (width 0.25) (layer "B.Cu") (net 5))
 (segment (start 84.1 111.7) (end 82.3 113.5) (width 0.25) (layer "B.Cu") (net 5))
 (segment (start 85.3 115.3) (end 87.5 113.1) (width 0.25) (layer "B.Cu") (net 5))
 (segment (start 83.4 104.5) (end 84.1 105.2) (width 0.25) (layer "B.Cu") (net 5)))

